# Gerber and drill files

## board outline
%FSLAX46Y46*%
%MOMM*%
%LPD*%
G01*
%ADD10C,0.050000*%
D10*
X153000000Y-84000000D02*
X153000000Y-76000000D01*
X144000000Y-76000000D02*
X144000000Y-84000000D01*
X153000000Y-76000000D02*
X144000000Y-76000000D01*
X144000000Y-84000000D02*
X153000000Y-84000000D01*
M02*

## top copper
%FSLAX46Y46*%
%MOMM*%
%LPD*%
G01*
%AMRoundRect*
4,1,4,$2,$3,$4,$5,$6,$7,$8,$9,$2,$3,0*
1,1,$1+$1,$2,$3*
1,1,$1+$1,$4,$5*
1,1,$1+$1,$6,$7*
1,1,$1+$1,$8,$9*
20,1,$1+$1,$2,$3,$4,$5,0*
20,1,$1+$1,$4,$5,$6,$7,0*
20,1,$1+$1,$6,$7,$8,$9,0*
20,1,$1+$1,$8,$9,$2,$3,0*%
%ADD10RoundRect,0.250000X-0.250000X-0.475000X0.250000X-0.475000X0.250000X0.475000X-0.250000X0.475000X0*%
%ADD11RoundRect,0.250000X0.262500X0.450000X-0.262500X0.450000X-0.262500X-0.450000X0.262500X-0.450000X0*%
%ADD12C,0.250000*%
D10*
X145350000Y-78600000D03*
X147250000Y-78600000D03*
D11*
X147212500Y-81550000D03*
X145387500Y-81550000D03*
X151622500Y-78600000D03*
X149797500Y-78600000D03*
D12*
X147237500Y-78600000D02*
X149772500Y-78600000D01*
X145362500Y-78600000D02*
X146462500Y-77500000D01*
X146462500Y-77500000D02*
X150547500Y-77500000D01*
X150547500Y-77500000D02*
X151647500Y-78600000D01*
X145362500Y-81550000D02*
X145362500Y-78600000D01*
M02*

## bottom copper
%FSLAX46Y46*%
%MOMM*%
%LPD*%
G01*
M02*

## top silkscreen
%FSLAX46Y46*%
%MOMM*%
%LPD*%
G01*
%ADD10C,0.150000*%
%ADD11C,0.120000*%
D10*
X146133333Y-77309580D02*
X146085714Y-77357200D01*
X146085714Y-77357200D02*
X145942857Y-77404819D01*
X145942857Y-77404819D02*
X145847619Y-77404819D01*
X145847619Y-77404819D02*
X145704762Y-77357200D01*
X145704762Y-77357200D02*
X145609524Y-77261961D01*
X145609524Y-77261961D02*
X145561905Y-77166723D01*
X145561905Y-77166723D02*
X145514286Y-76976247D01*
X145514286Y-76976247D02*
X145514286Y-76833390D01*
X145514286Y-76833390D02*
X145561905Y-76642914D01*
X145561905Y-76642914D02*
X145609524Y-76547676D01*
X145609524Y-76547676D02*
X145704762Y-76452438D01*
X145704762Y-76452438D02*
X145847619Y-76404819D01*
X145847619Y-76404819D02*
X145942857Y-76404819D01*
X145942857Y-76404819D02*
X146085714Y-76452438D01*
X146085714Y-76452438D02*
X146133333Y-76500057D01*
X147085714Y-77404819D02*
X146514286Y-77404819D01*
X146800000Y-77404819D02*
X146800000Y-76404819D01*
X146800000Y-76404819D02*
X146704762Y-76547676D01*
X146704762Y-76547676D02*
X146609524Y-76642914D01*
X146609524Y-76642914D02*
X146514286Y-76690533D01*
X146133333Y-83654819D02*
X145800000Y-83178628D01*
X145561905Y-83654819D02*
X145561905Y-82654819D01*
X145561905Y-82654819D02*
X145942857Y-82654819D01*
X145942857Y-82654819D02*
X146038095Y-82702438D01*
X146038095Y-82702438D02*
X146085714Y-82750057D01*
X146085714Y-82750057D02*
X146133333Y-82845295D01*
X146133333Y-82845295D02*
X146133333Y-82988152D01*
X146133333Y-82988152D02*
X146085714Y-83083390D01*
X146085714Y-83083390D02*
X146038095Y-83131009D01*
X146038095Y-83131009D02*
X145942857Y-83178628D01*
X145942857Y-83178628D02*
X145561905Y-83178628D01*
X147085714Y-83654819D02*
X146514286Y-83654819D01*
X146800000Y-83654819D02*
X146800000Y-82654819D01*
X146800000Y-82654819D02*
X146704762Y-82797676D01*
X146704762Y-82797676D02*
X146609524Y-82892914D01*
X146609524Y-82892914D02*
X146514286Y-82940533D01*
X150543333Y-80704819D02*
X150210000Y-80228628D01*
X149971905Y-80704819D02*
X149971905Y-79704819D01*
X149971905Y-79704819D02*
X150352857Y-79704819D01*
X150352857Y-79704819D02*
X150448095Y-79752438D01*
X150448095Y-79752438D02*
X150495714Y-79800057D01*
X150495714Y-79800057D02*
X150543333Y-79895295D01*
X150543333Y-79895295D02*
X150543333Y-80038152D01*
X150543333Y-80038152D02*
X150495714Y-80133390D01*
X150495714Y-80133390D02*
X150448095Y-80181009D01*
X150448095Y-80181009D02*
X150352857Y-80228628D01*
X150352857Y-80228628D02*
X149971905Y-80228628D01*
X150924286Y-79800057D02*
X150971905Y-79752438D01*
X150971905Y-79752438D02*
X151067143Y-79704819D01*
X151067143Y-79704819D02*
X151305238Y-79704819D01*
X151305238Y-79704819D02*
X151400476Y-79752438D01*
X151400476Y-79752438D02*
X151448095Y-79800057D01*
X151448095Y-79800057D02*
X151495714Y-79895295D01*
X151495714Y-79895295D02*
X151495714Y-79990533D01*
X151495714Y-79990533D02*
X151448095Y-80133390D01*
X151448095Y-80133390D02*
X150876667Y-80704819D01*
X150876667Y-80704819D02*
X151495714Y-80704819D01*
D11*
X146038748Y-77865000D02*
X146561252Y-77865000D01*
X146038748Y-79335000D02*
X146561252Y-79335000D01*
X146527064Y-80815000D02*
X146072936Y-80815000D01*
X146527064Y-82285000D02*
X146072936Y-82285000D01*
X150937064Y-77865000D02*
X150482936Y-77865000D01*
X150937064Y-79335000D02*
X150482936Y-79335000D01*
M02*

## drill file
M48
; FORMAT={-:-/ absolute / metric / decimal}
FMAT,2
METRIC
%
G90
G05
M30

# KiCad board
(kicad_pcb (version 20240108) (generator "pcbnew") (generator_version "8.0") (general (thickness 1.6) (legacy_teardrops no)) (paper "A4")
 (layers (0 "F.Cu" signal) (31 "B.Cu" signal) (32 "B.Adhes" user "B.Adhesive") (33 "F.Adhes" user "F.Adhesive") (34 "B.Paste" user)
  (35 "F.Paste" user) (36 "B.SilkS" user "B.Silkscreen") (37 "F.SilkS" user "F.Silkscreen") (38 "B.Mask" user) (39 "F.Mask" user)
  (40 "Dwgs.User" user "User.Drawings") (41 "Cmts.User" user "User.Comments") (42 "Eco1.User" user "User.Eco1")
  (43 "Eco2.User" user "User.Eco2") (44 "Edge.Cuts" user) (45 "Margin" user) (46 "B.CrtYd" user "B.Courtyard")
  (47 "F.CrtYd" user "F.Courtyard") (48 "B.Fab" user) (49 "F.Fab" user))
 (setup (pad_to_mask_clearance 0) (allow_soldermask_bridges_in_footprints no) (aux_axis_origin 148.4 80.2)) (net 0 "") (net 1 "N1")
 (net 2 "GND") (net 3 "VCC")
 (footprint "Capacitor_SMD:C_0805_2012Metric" (layer "F.Cu") (at 146.3 78.6)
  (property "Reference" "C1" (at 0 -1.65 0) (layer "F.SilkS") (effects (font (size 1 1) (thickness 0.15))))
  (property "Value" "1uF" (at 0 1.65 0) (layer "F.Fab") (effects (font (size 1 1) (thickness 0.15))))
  (fp_line (start -0.261252 -0.735) (end 0.261252 -0.735) (stroke (width 0.12) (type solid)) (layer "F.SilkS"))
  (fp_line (start -0.261252 0.735) (end 0.261252 0.735) (stroke (width 0.12) (type solid)) (layer "F.SilkS"))
  (pad "1" smd roundrect (at -0.95 0) (size 1 1.45) (layers "F.Cu" "F.Paste" "F.Mask") (roundrect_rratio 0.25) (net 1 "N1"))
  (pad "2" smd roundrect (at 0.95 0) (size 1 1.45) (layers "F.Cu" "F.Paste" "F.Mask") (roundrect_rratio 0.25) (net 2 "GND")))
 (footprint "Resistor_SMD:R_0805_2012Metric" (layer "F.Cu") (at 146.3 81.55 180)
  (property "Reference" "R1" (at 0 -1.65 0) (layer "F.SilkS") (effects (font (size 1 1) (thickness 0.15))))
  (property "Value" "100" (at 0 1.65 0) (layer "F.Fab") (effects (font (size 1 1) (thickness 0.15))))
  (fp_line (start -0.227064 0.735) (end 0.227064 0.735) (stroke (width 0.12) (type solid)) (layer "F.SilkS"))
  (fp_line (start -0.227064 -0.735) (end 0.227064 -0.735) (stroke (width 0.12) (type solid)) (layer "F.SilkS"))
  (pad "1" smd roundrect (at -0.9125 0 180) (size 1.025 1.4) (layers "F.Cu" "F.Paste" "F.Mask") (roundrect_rratio 0.243902) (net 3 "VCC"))
  (pad "2" smd roundrect (at 0.9125 0 180) (size 1.025 1.4) (layers "F.Cu" "F.Paste" "F.Mask") (roundrect_rratio 0.243902) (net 1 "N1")))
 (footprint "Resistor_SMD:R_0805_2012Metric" (layer "F.Cu") (at 150.71 78.6 180)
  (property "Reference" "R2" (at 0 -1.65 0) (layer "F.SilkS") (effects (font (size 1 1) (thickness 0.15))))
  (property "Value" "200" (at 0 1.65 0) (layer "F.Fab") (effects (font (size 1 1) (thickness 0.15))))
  (fp_line (start -0.227064 0.735) (end 0.227064 0.735) (stroke (width 0.12) (type solid)) (layer "F.SilkS"))
  (fp_line (start -0.227064 -0.735) (end 0.227064 -0.735) (stroke (width 0.12) (type solid)) (layer "F.SilkS"))
  (pad "1" smd roundrect (at -0.9125 0 180) (size 1.025 1.4) (layers "F.Cu" "F.Paste" "F.Mask") (roundrect_rratio 0.243902) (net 1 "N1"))
  (pad "2" smd roundrect (at 0.9125 0 180) (size 1.025 1.4) (layers "F.Cu" "F.Paste" "F.Mask") (roundrect_rratio 0.243902) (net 2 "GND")))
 (gr_line (start 153 84) (end 153 76) (stroke (width 0.05) (type solid)) (layer "Edge.Cuts"))
 (gr_line (start 144 76) (end 144 84) (stroke (width 0.05) (type solid)) (layer "Edge.Cuts"))
 (gr_line (start 153 76) (end 144 76) (stroke (width 0.05) (type solid)) (layer "Edge.Cuts"))
 (gr_line (start 144 84) (end 153 84) (stroke (width 0.05) (type solid)) (layer "Edge.Cuts"))
 (segment (start 147.2375 78.6) (end 149.7725 78.6) (width 0.25) (layer "F.Cu") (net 2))
 (segment (start 145.3625 78.6) (end 146.4625 77.5) (width 0.25) (layer "F.Cu") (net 1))
 (segment (start 146.4625 77.5) (end 150.5475 77.5) (width 0.25) (layer "F.Cu") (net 1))
 (segment (start 150.5475 77.5) (end 151.6475 78.6) (width 0.25) (layer "F.Cu") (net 1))
 (segment (start 145.3625 81.55) (end 145.3625 78.6) (width 0.25) (layer "F.Cu") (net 1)))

